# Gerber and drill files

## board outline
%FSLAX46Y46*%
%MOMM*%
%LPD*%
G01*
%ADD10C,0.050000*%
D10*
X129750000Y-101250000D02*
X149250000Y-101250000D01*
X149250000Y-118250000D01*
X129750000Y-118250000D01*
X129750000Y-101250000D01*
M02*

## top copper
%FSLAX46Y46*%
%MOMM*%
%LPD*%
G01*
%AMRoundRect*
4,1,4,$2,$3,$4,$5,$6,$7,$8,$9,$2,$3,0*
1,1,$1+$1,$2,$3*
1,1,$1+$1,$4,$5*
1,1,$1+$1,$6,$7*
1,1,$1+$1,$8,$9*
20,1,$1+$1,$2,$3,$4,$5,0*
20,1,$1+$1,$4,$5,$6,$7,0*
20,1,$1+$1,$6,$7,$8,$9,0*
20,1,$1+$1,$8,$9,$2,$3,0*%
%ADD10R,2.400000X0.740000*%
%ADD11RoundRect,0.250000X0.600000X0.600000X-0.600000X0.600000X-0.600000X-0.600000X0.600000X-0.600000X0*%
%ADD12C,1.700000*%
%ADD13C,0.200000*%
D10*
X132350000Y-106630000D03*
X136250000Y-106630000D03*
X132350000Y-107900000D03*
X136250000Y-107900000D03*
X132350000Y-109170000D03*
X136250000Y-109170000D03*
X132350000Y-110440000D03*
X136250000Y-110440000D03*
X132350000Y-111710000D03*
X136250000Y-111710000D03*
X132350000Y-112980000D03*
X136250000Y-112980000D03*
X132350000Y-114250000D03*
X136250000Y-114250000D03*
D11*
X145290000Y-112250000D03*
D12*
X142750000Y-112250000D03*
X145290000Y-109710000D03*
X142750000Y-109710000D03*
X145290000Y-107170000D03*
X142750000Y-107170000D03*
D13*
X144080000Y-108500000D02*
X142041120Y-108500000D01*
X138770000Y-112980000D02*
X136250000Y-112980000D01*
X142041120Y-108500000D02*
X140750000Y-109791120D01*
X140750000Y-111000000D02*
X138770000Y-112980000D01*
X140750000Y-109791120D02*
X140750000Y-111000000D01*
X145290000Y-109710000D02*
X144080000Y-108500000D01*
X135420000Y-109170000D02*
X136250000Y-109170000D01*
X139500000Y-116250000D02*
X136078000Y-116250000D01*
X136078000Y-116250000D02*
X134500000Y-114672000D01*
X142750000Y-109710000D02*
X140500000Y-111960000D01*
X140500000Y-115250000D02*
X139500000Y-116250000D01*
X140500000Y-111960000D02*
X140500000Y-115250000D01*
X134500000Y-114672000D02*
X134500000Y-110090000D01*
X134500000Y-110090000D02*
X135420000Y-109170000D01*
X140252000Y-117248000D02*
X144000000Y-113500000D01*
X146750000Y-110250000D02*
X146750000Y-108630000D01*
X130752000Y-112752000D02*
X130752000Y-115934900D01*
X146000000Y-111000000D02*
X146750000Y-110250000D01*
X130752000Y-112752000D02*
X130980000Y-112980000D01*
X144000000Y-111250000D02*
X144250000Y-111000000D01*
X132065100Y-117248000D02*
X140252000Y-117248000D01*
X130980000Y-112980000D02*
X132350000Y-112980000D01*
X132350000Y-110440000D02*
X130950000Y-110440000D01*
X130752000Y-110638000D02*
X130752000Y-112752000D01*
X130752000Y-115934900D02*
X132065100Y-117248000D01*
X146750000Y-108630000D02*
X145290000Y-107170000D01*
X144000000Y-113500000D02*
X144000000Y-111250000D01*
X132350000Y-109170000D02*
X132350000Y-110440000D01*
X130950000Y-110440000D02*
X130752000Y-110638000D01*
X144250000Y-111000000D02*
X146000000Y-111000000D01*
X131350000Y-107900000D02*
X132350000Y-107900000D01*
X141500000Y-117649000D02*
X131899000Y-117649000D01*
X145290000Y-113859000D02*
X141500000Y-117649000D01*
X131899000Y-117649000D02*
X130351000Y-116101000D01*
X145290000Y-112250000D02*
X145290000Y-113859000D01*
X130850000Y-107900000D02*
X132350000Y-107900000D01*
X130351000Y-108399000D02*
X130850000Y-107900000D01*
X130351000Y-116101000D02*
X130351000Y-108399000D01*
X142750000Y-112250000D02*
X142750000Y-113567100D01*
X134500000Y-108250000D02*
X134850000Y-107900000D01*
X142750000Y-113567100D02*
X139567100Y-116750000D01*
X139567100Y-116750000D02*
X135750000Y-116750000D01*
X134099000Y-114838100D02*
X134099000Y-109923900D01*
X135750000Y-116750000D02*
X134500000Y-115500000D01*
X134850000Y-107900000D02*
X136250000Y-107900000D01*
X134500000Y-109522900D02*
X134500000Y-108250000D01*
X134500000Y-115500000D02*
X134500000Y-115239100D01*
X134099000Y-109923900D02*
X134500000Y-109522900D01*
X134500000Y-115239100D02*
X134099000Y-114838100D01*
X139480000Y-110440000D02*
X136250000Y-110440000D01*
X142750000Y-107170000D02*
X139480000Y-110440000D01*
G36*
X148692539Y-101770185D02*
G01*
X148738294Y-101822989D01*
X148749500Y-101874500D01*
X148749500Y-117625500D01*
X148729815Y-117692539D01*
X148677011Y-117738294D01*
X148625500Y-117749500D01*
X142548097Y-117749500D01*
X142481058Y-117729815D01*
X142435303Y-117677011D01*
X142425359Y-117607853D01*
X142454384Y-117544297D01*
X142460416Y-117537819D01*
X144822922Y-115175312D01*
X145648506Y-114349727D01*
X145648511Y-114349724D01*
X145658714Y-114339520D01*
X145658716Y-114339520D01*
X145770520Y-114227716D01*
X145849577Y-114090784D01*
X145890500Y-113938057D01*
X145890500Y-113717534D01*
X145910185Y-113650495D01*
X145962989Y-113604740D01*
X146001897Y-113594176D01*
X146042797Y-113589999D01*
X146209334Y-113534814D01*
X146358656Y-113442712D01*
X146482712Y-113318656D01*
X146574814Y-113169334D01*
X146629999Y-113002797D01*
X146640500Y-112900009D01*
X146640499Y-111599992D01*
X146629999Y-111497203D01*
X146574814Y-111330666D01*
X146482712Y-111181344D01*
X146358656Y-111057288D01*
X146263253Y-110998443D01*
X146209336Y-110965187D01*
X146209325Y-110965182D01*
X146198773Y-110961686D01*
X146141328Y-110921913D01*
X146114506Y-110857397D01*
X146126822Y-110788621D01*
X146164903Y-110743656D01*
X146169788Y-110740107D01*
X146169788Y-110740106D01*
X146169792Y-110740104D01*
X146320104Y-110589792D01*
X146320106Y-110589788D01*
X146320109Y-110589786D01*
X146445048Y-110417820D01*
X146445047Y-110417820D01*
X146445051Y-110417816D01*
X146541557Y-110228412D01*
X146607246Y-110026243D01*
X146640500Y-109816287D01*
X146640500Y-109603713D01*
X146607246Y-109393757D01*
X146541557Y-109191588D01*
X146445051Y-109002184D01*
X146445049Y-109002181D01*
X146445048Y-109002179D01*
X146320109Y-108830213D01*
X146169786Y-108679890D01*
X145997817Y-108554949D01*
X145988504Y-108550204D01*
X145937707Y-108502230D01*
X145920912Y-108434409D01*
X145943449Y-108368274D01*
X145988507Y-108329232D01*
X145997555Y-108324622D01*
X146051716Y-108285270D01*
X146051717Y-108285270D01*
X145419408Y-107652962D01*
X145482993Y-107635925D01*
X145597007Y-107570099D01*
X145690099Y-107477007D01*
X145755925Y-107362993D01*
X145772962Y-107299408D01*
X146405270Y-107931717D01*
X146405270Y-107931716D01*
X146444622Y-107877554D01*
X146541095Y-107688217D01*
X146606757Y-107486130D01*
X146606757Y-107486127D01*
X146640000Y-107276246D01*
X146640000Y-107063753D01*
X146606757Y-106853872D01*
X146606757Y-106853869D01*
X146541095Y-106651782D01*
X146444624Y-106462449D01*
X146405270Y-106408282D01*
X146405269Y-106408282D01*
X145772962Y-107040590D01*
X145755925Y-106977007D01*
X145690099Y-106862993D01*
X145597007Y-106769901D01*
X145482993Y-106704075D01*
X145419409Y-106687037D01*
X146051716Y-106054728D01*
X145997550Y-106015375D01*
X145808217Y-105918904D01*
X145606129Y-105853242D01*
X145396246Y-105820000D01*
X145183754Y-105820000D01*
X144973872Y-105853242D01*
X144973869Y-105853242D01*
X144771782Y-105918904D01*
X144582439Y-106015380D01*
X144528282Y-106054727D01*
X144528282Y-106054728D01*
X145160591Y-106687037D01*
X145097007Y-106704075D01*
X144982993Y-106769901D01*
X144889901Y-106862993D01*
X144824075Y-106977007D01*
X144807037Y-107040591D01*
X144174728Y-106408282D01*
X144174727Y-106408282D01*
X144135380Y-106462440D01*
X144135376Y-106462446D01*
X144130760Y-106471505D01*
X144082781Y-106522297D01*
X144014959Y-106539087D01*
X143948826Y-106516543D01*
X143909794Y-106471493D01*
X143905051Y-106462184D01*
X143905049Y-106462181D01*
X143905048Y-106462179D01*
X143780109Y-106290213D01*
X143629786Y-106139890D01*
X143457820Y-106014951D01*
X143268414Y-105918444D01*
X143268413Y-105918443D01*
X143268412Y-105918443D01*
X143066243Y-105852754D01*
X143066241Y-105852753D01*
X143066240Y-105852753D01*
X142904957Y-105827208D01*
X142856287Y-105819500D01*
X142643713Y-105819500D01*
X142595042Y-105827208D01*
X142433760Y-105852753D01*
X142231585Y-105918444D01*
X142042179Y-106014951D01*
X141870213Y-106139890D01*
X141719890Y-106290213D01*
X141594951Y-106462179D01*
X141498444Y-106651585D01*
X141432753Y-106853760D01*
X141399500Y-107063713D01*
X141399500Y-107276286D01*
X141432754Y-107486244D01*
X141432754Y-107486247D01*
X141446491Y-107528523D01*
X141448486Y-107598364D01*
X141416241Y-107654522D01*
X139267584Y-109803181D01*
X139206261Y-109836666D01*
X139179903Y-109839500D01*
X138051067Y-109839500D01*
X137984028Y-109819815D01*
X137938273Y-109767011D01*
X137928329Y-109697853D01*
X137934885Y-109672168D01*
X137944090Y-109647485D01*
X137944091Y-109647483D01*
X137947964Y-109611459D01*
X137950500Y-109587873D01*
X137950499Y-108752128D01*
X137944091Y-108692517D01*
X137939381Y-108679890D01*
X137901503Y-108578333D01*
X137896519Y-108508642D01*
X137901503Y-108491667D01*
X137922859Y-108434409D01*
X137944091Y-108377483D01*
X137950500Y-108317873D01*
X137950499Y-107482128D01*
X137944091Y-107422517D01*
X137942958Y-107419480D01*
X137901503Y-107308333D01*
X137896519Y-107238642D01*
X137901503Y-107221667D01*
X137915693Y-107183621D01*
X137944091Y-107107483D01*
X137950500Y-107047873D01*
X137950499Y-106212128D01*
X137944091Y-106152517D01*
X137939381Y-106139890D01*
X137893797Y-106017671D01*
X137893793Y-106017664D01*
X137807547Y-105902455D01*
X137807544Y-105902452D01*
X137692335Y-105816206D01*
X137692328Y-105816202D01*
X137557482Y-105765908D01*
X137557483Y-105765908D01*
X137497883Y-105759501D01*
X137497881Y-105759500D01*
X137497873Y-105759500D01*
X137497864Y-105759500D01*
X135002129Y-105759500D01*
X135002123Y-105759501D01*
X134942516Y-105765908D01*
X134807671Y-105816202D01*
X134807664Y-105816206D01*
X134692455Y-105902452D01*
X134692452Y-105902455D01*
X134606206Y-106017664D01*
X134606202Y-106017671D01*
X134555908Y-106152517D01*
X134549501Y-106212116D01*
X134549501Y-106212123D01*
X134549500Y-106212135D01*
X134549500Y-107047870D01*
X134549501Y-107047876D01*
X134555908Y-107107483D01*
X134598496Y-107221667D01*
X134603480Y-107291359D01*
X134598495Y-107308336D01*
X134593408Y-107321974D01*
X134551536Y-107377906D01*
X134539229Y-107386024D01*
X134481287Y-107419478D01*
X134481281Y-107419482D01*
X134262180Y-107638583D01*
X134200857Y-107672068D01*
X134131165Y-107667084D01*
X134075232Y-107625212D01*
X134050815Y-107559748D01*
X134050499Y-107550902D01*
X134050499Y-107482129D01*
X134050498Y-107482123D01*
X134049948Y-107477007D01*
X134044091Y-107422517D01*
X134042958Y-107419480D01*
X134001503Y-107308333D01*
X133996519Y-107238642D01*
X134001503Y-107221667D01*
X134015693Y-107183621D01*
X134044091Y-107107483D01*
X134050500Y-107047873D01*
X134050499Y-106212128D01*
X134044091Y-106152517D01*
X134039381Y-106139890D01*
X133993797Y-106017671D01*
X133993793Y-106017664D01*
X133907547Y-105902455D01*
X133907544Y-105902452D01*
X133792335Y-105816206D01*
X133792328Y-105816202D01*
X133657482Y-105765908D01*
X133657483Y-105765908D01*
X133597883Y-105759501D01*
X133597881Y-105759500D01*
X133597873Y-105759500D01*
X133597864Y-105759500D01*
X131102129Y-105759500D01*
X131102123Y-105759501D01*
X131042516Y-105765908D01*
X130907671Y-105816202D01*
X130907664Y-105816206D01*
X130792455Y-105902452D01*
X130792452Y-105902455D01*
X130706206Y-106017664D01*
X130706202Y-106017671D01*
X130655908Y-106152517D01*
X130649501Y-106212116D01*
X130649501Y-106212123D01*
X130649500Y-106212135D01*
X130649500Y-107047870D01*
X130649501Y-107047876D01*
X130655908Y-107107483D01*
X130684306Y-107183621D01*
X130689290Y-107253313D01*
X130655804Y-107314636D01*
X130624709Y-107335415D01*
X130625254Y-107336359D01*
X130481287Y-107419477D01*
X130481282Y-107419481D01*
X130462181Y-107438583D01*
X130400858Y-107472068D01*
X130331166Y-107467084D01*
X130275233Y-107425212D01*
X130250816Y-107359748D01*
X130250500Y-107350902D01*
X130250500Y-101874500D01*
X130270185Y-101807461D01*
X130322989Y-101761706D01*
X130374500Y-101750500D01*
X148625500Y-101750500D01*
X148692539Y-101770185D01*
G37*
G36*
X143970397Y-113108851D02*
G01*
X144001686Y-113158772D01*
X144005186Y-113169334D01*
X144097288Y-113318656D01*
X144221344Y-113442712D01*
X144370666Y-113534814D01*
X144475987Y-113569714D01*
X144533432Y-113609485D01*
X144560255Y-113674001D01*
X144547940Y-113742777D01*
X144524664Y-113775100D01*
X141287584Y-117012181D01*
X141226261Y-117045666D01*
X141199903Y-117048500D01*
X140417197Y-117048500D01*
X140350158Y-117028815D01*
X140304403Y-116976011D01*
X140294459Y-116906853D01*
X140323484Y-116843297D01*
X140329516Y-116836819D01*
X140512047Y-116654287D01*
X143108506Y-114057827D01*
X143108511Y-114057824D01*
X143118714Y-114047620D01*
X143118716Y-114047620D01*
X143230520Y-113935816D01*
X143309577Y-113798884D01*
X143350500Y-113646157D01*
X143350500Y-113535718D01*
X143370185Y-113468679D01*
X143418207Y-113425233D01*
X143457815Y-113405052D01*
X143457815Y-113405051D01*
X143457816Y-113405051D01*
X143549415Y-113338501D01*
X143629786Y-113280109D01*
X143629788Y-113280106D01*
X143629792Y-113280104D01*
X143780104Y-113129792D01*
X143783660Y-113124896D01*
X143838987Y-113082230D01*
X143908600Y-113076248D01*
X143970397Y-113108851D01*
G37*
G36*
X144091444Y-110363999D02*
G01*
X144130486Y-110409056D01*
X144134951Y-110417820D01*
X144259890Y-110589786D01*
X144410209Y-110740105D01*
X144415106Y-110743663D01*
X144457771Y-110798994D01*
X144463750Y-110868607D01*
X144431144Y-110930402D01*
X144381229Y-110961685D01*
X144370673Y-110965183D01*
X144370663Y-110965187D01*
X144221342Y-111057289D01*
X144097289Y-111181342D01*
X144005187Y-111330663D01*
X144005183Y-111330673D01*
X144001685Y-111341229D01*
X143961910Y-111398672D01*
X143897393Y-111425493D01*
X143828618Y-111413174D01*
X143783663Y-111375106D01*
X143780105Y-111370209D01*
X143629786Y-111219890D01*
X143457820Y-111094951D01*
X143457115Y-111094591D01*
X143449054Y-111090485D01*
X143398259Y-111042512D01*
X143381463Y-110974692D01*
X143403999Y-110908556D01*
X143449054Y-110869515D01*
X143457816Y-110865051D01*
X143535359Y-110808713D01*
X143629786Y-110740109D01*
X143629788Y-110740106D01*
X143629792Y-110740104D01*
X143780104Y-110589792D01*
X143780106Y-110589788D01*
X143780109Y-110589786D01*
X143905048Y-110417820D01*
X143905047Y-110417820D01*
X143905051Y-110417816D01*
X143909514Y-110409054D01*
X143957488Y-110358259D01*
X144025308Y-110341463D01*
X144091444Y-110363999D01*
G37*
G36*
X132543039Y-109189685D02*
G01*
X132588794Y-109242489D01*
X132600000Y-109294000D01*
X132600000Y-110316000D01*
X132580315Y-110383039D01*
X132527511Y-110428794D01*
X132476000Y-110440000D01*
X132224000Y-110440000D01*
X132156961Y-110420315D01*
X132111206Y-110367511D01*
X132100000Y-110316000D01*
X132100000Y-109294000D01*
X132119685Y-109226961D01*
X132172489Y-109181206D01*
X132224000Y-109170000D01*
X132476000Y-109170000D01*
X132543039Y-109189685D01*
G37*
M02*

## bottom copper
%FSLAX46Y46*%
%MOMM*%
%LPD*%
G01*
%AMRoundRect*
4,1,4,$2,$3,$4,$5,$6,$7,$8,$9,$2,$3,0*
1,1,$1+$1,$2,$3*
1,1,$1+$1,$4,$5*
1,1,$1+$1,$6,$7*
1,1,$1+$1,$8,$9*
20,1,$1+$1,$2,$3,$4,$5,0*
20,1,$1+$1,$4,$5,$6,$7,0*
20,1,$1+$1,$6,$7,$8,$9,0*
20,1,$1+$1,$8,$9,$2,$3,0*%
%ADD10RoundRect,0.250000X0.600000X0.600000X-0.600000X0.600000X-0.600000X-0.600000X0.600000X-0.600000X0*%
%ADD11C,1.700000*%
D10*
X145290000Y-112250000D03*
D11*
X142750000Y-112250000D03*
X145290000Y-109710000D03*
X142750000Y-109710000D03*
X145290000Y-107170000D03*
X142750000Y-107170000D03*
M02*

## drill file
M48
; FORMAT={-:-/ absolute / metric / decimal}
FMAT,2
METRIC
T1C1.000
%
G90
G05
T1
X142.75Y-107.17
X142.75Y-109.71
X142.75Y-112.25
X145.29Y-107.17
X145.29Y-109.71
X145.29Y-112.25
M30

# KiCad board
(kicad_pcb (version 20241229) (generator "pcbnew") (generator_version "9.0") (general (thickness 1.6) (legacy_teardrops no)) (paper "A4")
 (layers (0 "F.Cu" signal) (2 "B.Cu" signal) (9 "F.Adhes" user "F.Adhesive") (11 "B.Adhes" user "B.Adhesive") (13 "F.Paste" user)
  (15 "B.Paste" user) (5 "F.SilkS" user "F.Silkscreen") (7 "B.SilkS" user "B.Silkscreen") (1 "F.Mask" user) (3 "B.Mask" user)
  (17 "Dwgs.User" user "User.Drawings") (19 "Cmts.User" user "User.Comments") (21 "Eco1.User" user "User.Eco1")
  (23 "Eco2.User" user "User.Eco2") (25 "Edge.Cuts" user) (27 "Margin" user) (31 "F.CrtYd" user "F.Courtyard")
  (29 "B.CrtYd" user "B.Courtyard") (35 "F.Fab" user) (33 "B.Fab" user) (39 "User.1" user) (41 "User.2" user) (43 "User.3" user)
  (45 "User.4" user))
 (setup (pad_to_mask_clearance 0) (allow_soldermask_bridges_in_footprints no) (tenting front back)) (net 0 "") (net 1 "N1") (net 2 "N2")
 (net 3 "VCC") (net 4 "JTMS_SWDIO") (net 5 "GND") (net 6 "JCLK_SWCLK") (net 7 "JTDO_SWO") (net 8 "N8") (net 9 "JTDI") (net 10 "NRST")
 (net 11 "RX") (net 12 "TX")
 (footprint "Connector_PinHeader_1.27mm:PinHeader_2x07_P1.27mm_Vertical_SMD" (layer "F.Cu") (at 134.3 110.44)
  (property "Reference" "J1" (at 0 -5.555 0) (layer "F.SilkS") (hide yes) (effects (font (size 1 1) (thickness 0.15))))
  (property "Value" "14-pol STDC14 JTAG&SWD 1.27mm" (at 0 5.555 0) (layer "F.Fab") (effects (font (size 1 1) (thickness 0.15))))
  (pad "1" smd rect (at -1.95 -3.81) (size 2.4 0.74) (layers "F.Cu" "F.Mask" "F.Paste") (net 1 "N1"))
  (pad "2" smd rect (at 1.95 -3.81) (size 2.4 0.74) (layers "F.Cu" "F.Mask" "F.Paste") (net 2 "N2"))
  (pad "3" smd rect (at -1.95 -2.54) (size 2.4 0.74) (layers "F.Cu" "F.Mask" "F.Paste") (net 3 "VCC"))
  (pad "4" smd rect (at 1.95 -2.54) (size 2.4 0.74) (layers "F.Cu" "F.Mask" "F.Paste") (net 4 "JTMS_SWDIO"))
  (pad "5" smd rect (at -1.95 -1.27) (size 2.4 0.74) (layers "F.Cu" "F.Mask" "F.Paste") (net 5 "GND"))
  (pad "6" smd rect (at 1.95 -1.27) (size 2.4 0.74) (layers "F.Cu" "F.Mask" "F.Paste") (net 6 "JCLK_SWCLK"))
  (pad "7" smd rect (at -1.95 0) (size 2.4 0.74) (layers "F.Cu" "F.Mask" "F.Paste") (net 5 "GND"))
  (pad "8" smd rect (at 1.95 0) (size 2.4 0.74) (layers "F.Cu" "F.Mask" "F.Paste") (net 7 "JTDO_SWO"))
  (pad "9" smd rect (at -1.95 1.27) (size 2.4 0.74) (layers "F.Cu" "F.Mask" "F.Paste") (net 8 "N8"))
  (pad "10" smd rect (at 1.95 1.27) (size 2.4 0.74) (layers "F.Cu" "F.Mask" "F.Paste") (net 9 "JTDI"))
  (pad "11" smd rect (at -1.95 2.54) (size 2.4 0.74) (layers "F.Cu" "F.Mask" "F.Paste") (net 5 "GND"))
  (pad "12" smd rect (at 1.95 2.54) (size 2.4 0.74) (layers "F.Cu" "F.Mask" "F.Paste") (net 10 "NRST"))
  (pad "13" smd rect (at -1.95 3.81) (size 2.4 0.74) (layers "F.Cu" "F.Mask" "F.Paste") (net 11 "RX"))
  (pad "14" smd rect (at 1.95 3.81) (size 2.4 0.74) (layers "F.Cu" "F.Mask" "F.Paste") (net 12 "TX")))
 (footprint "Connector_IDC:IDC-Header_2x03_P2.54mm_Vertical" (layer "F.Cu") (at 145.29 112.25 180)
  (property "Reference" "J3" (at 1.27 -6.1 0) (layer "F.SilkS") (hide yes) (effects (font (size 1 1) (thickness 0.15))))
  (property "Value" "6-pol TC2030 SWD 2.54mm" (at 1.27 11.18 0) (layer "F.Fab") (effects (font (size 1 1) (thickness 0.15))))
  (pad "1" thru_hole roundrect (at 0 0 180) (size 1.7 1.7) (drill 1) (layers "*.Cu" "*.Mask") (remove_unused_layers no)
   (roundrect_rratio 0.147059) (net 3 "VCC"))
  (pad "2" thru_hole circle (at 2.54 0 180) (size 1.7 1.7) (drill 1) (layers "*.Cu" "*.Mask") (remove_unused_layers no) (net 4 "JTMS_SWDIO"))
  (pad "3" thru_hole circle (at 0 2.54 180) (size 1.7 1.7) (drill 1) (layers "*.Cu" "*.Mask") (remove_unused_layers no) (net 10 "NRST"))
  (pad "4" thru_hole circle (at 2.54 2.54 180) (size 1.7 1.7) (drill 1) (layers "*.Cu" "*.Mask") (remove_unused_layers no)
   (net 6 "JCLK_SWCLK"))
  (pad "5" thru_hole circle (at 0 5.08 180) (size 1.7 1.7) (drill 1) (layers "*.Cu" "*.Mask") (remove_unused_layers no) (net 5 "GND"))
  (pad "6" thru_hole circle (at 2.54 5.08 180) (size 1.7 1.7) (drill 1) (layers "*.Cu" "*.Mask") (remove_unused_layers no)
   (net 7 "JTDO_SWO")))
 (gr_rect (start 129.75 101.25) (end 149.25 118.25) (stroke (width 0.05) (type default)) (fill no) (layer "Edge.Cuts"))
 (segment (start 144.08 108.5) (end 142.04112 108.5) (width 0.2) (layer "F.Cu") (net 10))
 (segment (start 138.77 112.98) (end 136.25 112.98) (width 0.2) (layer "F.Cu") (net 10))
 (segment (start 142.04112 108.5) (end 140.75 109.79112) (width 0.2) (layer "F.Cu") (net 10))
 (segment (start 140.75 111) (end 138.77 112.98) (width 0.2) (layer "F.Cu") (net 10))
 (segment (start 140.75 109.79112) (end 140.75 111) (width 0.2) (layer "F.Cu") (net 10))
 (segment (start 145.29 109.71) (end 144.08 108.5) (width 0.2) (layer "F.Cu") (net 10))
 (segment (start 135.42 109.17) (end 136.25 109.17) (width 0.2) (layer "F.Cu") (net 6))
 (segment (start 139.5 116.25) (end 136.078 116.25) (width 0.2) (layer "F.Cu") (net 6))
 (segment (start 136.078 116.25) (end 134.5 114.672) (width 0.2) (layer "F.Cu") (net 6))
 (segment (start 142.75 109.71) (end 140.5 111.96) (width 0.2) (layer "F.Cu") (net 6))
 (segment (start 140.5 115.25) (end 139.5 116.25) (width 0.2) (layer "F.Cu") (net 6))
 (segment (start 140.5 111.96) (end 140.5 115.25) (width 0.2) (layer "F.Cu") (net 6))
 (segment (start 134.5 114.672) (end 134.5 110.09) (width 0.2) (layer "F.Cu") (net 6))
 (segment (start 134.5 110.09) (end 135.42 109.17) (width 0.2) (layer "F.Cu") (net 6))
 (segment (start 140.252 117.248) (end 144 113.5) (width 0.2) (layer "F.Cu") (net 5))
 (segment (start 146.75 110.25) (end 146.75 108.63) (width 0.2) (layer "F.Cu") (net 5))
 (segment (start 130.752 112.752) (end 130.752 115.9349) (width 0.2) (layer "F.Cu") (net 5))
 (segment (start 146 111) (end 146.75 110.25) (width 0.2) (layer "F.Cu") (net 5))
 (segment (start 130.752 112.752) (end 130.98 112.98) (width 0.2) (layer "F.Cu") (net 5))
 (segment (start 144 111.25) (end 144.25 111) (width 0.2) (layer "F.Cu") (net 5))
 (segment (start 132.0651 117.248) (end 140.252 117.248) (width 0.2) (layer "F.Cu") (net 5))
 (segment (start 130.98 112.98) (end 132.35 112.98) (width 0.2) (layer "F.Cu") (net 5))
 (segment (start 132.35 110.44) (end 130.95 110.44) (width 0.2) (layer "F.Cu") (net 5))
 (segment (start 130.752 110.638) (end 130.752 112.752) (width 0.2) (layer "F.Cu") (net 5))
 (segment (start 130.752 115.9349) (end 132.0651 117.248) (width 0.2) (layer "F.Cu") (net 5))
 (segment (start 146.75 108.63) (end 145.29 107.17) (width 0.2) (layer "F.Cu") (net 5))
 (segment (start 144 113.5) (end 144 111.25) (width 0.2) (layer "F.Cu") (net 5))
 (segment (start 132.35 109.17) (end 132.35 110.44) (width 0.2) (layer "F.Cu") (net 5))
 (segment (start 130.95 110.44) (end 130.752 110.638) (width 0.2) (layer "F.Cu") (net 5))
 (segment (start 144.25 111) (end 146 111) (width 0.2) (layer "F.Cu") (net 5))
 (segment (start 131.35 107.9) (end 132.35 107.9) (width 0.2) (layer "F.Cu") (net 3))
 (segment (start 141.5 117.649) (end 131.899 117.649) (width 0.2) (layer "F.Cu") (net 3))
 (segment (start 145.29 113.859) (end 141.5 117.649) (width 0.2) (layer "F.Cu") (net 3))
 (segment (start 131.899 117.649) (end 130.351 116.101) (width 0.2) (layer "F.Cu") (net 3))
 (segment (start 145.29 112.25) (end 145.29 113.859) (width 0.2) (layer "F.Cu") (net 3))
 (segment (start 130.85 107.9) (end 132.35 107.9) (width 0.2) (layer "F.Cu") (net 3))
 (segment (start 130.351 108.399) (end 130.85 107.9) (width 0.2) (layer "F.Cu") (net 3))
 (segment (start 130.351 116.101) (end 130.351 108.399) (width 0.2) (layer "F.Cu") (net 3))
 (segment (start 142.75 112.25) (end 142.75 113.5671) (width 0.2) (layer "F.Cu") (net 4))
 (segment (start 134.5 108.25) (end 134.85 107.9) (width 0.2) (layer "F.Cu") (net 4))
 (segment (start 142.75 113.5671) (end 139.5671 116.75) (width 0.2) (layer "F.Cu") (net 4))
 (segment (start 139.5671 116.75) (end 135.75 116.75) (width 0.2) (layer "F.Cu") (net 4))
 (segment (start 134.099 114.8381) (end 134.099 109.9239) (width 0.2) (layer "F.Cu") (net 4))
 (segment (start 135.75 116.75) (end 134.5 115.5) (width 0.2) (layer "F.Cu") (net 4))
 (segment (start 134.85 107.9) (end 136.25 107.9) (width 0.2) (layer "F.Cu") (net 4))
 (segment (start 134.5 109.5229) (end 134.5 108.25) (width 0.2) (layer "F.Cu") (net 4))
 (segment (start 134.5 115.5) (end 134.5 115.2391) (width 0.2) (layer "F.Cu") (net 4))
 (segment (start 134.099 109.9239) (end 134.5 109.5229) (width 0.2) (layer "F.Cu") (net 4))
 (segment (start 134.5 115.2391) (end 134.099 114.8381) (width 0.2) (layer "F.Cu") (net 4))
 (segment (start 139.48 110.44) (end 136.25 110.44) (width 0.2) (layer "F.Cu") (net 7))
 (segment (start 142.75 107.17) (end 139.48 110.44) (width 0.2) (layer "F.Cu") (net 7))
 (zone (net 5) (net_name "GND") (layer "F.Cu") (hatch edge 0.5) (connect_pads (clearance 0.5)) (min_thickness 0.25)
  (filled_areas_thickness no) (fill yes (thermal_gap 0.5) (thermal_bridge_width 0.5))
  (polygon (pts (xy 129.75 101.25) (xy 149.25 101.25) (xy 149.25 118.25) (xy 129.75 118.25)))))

